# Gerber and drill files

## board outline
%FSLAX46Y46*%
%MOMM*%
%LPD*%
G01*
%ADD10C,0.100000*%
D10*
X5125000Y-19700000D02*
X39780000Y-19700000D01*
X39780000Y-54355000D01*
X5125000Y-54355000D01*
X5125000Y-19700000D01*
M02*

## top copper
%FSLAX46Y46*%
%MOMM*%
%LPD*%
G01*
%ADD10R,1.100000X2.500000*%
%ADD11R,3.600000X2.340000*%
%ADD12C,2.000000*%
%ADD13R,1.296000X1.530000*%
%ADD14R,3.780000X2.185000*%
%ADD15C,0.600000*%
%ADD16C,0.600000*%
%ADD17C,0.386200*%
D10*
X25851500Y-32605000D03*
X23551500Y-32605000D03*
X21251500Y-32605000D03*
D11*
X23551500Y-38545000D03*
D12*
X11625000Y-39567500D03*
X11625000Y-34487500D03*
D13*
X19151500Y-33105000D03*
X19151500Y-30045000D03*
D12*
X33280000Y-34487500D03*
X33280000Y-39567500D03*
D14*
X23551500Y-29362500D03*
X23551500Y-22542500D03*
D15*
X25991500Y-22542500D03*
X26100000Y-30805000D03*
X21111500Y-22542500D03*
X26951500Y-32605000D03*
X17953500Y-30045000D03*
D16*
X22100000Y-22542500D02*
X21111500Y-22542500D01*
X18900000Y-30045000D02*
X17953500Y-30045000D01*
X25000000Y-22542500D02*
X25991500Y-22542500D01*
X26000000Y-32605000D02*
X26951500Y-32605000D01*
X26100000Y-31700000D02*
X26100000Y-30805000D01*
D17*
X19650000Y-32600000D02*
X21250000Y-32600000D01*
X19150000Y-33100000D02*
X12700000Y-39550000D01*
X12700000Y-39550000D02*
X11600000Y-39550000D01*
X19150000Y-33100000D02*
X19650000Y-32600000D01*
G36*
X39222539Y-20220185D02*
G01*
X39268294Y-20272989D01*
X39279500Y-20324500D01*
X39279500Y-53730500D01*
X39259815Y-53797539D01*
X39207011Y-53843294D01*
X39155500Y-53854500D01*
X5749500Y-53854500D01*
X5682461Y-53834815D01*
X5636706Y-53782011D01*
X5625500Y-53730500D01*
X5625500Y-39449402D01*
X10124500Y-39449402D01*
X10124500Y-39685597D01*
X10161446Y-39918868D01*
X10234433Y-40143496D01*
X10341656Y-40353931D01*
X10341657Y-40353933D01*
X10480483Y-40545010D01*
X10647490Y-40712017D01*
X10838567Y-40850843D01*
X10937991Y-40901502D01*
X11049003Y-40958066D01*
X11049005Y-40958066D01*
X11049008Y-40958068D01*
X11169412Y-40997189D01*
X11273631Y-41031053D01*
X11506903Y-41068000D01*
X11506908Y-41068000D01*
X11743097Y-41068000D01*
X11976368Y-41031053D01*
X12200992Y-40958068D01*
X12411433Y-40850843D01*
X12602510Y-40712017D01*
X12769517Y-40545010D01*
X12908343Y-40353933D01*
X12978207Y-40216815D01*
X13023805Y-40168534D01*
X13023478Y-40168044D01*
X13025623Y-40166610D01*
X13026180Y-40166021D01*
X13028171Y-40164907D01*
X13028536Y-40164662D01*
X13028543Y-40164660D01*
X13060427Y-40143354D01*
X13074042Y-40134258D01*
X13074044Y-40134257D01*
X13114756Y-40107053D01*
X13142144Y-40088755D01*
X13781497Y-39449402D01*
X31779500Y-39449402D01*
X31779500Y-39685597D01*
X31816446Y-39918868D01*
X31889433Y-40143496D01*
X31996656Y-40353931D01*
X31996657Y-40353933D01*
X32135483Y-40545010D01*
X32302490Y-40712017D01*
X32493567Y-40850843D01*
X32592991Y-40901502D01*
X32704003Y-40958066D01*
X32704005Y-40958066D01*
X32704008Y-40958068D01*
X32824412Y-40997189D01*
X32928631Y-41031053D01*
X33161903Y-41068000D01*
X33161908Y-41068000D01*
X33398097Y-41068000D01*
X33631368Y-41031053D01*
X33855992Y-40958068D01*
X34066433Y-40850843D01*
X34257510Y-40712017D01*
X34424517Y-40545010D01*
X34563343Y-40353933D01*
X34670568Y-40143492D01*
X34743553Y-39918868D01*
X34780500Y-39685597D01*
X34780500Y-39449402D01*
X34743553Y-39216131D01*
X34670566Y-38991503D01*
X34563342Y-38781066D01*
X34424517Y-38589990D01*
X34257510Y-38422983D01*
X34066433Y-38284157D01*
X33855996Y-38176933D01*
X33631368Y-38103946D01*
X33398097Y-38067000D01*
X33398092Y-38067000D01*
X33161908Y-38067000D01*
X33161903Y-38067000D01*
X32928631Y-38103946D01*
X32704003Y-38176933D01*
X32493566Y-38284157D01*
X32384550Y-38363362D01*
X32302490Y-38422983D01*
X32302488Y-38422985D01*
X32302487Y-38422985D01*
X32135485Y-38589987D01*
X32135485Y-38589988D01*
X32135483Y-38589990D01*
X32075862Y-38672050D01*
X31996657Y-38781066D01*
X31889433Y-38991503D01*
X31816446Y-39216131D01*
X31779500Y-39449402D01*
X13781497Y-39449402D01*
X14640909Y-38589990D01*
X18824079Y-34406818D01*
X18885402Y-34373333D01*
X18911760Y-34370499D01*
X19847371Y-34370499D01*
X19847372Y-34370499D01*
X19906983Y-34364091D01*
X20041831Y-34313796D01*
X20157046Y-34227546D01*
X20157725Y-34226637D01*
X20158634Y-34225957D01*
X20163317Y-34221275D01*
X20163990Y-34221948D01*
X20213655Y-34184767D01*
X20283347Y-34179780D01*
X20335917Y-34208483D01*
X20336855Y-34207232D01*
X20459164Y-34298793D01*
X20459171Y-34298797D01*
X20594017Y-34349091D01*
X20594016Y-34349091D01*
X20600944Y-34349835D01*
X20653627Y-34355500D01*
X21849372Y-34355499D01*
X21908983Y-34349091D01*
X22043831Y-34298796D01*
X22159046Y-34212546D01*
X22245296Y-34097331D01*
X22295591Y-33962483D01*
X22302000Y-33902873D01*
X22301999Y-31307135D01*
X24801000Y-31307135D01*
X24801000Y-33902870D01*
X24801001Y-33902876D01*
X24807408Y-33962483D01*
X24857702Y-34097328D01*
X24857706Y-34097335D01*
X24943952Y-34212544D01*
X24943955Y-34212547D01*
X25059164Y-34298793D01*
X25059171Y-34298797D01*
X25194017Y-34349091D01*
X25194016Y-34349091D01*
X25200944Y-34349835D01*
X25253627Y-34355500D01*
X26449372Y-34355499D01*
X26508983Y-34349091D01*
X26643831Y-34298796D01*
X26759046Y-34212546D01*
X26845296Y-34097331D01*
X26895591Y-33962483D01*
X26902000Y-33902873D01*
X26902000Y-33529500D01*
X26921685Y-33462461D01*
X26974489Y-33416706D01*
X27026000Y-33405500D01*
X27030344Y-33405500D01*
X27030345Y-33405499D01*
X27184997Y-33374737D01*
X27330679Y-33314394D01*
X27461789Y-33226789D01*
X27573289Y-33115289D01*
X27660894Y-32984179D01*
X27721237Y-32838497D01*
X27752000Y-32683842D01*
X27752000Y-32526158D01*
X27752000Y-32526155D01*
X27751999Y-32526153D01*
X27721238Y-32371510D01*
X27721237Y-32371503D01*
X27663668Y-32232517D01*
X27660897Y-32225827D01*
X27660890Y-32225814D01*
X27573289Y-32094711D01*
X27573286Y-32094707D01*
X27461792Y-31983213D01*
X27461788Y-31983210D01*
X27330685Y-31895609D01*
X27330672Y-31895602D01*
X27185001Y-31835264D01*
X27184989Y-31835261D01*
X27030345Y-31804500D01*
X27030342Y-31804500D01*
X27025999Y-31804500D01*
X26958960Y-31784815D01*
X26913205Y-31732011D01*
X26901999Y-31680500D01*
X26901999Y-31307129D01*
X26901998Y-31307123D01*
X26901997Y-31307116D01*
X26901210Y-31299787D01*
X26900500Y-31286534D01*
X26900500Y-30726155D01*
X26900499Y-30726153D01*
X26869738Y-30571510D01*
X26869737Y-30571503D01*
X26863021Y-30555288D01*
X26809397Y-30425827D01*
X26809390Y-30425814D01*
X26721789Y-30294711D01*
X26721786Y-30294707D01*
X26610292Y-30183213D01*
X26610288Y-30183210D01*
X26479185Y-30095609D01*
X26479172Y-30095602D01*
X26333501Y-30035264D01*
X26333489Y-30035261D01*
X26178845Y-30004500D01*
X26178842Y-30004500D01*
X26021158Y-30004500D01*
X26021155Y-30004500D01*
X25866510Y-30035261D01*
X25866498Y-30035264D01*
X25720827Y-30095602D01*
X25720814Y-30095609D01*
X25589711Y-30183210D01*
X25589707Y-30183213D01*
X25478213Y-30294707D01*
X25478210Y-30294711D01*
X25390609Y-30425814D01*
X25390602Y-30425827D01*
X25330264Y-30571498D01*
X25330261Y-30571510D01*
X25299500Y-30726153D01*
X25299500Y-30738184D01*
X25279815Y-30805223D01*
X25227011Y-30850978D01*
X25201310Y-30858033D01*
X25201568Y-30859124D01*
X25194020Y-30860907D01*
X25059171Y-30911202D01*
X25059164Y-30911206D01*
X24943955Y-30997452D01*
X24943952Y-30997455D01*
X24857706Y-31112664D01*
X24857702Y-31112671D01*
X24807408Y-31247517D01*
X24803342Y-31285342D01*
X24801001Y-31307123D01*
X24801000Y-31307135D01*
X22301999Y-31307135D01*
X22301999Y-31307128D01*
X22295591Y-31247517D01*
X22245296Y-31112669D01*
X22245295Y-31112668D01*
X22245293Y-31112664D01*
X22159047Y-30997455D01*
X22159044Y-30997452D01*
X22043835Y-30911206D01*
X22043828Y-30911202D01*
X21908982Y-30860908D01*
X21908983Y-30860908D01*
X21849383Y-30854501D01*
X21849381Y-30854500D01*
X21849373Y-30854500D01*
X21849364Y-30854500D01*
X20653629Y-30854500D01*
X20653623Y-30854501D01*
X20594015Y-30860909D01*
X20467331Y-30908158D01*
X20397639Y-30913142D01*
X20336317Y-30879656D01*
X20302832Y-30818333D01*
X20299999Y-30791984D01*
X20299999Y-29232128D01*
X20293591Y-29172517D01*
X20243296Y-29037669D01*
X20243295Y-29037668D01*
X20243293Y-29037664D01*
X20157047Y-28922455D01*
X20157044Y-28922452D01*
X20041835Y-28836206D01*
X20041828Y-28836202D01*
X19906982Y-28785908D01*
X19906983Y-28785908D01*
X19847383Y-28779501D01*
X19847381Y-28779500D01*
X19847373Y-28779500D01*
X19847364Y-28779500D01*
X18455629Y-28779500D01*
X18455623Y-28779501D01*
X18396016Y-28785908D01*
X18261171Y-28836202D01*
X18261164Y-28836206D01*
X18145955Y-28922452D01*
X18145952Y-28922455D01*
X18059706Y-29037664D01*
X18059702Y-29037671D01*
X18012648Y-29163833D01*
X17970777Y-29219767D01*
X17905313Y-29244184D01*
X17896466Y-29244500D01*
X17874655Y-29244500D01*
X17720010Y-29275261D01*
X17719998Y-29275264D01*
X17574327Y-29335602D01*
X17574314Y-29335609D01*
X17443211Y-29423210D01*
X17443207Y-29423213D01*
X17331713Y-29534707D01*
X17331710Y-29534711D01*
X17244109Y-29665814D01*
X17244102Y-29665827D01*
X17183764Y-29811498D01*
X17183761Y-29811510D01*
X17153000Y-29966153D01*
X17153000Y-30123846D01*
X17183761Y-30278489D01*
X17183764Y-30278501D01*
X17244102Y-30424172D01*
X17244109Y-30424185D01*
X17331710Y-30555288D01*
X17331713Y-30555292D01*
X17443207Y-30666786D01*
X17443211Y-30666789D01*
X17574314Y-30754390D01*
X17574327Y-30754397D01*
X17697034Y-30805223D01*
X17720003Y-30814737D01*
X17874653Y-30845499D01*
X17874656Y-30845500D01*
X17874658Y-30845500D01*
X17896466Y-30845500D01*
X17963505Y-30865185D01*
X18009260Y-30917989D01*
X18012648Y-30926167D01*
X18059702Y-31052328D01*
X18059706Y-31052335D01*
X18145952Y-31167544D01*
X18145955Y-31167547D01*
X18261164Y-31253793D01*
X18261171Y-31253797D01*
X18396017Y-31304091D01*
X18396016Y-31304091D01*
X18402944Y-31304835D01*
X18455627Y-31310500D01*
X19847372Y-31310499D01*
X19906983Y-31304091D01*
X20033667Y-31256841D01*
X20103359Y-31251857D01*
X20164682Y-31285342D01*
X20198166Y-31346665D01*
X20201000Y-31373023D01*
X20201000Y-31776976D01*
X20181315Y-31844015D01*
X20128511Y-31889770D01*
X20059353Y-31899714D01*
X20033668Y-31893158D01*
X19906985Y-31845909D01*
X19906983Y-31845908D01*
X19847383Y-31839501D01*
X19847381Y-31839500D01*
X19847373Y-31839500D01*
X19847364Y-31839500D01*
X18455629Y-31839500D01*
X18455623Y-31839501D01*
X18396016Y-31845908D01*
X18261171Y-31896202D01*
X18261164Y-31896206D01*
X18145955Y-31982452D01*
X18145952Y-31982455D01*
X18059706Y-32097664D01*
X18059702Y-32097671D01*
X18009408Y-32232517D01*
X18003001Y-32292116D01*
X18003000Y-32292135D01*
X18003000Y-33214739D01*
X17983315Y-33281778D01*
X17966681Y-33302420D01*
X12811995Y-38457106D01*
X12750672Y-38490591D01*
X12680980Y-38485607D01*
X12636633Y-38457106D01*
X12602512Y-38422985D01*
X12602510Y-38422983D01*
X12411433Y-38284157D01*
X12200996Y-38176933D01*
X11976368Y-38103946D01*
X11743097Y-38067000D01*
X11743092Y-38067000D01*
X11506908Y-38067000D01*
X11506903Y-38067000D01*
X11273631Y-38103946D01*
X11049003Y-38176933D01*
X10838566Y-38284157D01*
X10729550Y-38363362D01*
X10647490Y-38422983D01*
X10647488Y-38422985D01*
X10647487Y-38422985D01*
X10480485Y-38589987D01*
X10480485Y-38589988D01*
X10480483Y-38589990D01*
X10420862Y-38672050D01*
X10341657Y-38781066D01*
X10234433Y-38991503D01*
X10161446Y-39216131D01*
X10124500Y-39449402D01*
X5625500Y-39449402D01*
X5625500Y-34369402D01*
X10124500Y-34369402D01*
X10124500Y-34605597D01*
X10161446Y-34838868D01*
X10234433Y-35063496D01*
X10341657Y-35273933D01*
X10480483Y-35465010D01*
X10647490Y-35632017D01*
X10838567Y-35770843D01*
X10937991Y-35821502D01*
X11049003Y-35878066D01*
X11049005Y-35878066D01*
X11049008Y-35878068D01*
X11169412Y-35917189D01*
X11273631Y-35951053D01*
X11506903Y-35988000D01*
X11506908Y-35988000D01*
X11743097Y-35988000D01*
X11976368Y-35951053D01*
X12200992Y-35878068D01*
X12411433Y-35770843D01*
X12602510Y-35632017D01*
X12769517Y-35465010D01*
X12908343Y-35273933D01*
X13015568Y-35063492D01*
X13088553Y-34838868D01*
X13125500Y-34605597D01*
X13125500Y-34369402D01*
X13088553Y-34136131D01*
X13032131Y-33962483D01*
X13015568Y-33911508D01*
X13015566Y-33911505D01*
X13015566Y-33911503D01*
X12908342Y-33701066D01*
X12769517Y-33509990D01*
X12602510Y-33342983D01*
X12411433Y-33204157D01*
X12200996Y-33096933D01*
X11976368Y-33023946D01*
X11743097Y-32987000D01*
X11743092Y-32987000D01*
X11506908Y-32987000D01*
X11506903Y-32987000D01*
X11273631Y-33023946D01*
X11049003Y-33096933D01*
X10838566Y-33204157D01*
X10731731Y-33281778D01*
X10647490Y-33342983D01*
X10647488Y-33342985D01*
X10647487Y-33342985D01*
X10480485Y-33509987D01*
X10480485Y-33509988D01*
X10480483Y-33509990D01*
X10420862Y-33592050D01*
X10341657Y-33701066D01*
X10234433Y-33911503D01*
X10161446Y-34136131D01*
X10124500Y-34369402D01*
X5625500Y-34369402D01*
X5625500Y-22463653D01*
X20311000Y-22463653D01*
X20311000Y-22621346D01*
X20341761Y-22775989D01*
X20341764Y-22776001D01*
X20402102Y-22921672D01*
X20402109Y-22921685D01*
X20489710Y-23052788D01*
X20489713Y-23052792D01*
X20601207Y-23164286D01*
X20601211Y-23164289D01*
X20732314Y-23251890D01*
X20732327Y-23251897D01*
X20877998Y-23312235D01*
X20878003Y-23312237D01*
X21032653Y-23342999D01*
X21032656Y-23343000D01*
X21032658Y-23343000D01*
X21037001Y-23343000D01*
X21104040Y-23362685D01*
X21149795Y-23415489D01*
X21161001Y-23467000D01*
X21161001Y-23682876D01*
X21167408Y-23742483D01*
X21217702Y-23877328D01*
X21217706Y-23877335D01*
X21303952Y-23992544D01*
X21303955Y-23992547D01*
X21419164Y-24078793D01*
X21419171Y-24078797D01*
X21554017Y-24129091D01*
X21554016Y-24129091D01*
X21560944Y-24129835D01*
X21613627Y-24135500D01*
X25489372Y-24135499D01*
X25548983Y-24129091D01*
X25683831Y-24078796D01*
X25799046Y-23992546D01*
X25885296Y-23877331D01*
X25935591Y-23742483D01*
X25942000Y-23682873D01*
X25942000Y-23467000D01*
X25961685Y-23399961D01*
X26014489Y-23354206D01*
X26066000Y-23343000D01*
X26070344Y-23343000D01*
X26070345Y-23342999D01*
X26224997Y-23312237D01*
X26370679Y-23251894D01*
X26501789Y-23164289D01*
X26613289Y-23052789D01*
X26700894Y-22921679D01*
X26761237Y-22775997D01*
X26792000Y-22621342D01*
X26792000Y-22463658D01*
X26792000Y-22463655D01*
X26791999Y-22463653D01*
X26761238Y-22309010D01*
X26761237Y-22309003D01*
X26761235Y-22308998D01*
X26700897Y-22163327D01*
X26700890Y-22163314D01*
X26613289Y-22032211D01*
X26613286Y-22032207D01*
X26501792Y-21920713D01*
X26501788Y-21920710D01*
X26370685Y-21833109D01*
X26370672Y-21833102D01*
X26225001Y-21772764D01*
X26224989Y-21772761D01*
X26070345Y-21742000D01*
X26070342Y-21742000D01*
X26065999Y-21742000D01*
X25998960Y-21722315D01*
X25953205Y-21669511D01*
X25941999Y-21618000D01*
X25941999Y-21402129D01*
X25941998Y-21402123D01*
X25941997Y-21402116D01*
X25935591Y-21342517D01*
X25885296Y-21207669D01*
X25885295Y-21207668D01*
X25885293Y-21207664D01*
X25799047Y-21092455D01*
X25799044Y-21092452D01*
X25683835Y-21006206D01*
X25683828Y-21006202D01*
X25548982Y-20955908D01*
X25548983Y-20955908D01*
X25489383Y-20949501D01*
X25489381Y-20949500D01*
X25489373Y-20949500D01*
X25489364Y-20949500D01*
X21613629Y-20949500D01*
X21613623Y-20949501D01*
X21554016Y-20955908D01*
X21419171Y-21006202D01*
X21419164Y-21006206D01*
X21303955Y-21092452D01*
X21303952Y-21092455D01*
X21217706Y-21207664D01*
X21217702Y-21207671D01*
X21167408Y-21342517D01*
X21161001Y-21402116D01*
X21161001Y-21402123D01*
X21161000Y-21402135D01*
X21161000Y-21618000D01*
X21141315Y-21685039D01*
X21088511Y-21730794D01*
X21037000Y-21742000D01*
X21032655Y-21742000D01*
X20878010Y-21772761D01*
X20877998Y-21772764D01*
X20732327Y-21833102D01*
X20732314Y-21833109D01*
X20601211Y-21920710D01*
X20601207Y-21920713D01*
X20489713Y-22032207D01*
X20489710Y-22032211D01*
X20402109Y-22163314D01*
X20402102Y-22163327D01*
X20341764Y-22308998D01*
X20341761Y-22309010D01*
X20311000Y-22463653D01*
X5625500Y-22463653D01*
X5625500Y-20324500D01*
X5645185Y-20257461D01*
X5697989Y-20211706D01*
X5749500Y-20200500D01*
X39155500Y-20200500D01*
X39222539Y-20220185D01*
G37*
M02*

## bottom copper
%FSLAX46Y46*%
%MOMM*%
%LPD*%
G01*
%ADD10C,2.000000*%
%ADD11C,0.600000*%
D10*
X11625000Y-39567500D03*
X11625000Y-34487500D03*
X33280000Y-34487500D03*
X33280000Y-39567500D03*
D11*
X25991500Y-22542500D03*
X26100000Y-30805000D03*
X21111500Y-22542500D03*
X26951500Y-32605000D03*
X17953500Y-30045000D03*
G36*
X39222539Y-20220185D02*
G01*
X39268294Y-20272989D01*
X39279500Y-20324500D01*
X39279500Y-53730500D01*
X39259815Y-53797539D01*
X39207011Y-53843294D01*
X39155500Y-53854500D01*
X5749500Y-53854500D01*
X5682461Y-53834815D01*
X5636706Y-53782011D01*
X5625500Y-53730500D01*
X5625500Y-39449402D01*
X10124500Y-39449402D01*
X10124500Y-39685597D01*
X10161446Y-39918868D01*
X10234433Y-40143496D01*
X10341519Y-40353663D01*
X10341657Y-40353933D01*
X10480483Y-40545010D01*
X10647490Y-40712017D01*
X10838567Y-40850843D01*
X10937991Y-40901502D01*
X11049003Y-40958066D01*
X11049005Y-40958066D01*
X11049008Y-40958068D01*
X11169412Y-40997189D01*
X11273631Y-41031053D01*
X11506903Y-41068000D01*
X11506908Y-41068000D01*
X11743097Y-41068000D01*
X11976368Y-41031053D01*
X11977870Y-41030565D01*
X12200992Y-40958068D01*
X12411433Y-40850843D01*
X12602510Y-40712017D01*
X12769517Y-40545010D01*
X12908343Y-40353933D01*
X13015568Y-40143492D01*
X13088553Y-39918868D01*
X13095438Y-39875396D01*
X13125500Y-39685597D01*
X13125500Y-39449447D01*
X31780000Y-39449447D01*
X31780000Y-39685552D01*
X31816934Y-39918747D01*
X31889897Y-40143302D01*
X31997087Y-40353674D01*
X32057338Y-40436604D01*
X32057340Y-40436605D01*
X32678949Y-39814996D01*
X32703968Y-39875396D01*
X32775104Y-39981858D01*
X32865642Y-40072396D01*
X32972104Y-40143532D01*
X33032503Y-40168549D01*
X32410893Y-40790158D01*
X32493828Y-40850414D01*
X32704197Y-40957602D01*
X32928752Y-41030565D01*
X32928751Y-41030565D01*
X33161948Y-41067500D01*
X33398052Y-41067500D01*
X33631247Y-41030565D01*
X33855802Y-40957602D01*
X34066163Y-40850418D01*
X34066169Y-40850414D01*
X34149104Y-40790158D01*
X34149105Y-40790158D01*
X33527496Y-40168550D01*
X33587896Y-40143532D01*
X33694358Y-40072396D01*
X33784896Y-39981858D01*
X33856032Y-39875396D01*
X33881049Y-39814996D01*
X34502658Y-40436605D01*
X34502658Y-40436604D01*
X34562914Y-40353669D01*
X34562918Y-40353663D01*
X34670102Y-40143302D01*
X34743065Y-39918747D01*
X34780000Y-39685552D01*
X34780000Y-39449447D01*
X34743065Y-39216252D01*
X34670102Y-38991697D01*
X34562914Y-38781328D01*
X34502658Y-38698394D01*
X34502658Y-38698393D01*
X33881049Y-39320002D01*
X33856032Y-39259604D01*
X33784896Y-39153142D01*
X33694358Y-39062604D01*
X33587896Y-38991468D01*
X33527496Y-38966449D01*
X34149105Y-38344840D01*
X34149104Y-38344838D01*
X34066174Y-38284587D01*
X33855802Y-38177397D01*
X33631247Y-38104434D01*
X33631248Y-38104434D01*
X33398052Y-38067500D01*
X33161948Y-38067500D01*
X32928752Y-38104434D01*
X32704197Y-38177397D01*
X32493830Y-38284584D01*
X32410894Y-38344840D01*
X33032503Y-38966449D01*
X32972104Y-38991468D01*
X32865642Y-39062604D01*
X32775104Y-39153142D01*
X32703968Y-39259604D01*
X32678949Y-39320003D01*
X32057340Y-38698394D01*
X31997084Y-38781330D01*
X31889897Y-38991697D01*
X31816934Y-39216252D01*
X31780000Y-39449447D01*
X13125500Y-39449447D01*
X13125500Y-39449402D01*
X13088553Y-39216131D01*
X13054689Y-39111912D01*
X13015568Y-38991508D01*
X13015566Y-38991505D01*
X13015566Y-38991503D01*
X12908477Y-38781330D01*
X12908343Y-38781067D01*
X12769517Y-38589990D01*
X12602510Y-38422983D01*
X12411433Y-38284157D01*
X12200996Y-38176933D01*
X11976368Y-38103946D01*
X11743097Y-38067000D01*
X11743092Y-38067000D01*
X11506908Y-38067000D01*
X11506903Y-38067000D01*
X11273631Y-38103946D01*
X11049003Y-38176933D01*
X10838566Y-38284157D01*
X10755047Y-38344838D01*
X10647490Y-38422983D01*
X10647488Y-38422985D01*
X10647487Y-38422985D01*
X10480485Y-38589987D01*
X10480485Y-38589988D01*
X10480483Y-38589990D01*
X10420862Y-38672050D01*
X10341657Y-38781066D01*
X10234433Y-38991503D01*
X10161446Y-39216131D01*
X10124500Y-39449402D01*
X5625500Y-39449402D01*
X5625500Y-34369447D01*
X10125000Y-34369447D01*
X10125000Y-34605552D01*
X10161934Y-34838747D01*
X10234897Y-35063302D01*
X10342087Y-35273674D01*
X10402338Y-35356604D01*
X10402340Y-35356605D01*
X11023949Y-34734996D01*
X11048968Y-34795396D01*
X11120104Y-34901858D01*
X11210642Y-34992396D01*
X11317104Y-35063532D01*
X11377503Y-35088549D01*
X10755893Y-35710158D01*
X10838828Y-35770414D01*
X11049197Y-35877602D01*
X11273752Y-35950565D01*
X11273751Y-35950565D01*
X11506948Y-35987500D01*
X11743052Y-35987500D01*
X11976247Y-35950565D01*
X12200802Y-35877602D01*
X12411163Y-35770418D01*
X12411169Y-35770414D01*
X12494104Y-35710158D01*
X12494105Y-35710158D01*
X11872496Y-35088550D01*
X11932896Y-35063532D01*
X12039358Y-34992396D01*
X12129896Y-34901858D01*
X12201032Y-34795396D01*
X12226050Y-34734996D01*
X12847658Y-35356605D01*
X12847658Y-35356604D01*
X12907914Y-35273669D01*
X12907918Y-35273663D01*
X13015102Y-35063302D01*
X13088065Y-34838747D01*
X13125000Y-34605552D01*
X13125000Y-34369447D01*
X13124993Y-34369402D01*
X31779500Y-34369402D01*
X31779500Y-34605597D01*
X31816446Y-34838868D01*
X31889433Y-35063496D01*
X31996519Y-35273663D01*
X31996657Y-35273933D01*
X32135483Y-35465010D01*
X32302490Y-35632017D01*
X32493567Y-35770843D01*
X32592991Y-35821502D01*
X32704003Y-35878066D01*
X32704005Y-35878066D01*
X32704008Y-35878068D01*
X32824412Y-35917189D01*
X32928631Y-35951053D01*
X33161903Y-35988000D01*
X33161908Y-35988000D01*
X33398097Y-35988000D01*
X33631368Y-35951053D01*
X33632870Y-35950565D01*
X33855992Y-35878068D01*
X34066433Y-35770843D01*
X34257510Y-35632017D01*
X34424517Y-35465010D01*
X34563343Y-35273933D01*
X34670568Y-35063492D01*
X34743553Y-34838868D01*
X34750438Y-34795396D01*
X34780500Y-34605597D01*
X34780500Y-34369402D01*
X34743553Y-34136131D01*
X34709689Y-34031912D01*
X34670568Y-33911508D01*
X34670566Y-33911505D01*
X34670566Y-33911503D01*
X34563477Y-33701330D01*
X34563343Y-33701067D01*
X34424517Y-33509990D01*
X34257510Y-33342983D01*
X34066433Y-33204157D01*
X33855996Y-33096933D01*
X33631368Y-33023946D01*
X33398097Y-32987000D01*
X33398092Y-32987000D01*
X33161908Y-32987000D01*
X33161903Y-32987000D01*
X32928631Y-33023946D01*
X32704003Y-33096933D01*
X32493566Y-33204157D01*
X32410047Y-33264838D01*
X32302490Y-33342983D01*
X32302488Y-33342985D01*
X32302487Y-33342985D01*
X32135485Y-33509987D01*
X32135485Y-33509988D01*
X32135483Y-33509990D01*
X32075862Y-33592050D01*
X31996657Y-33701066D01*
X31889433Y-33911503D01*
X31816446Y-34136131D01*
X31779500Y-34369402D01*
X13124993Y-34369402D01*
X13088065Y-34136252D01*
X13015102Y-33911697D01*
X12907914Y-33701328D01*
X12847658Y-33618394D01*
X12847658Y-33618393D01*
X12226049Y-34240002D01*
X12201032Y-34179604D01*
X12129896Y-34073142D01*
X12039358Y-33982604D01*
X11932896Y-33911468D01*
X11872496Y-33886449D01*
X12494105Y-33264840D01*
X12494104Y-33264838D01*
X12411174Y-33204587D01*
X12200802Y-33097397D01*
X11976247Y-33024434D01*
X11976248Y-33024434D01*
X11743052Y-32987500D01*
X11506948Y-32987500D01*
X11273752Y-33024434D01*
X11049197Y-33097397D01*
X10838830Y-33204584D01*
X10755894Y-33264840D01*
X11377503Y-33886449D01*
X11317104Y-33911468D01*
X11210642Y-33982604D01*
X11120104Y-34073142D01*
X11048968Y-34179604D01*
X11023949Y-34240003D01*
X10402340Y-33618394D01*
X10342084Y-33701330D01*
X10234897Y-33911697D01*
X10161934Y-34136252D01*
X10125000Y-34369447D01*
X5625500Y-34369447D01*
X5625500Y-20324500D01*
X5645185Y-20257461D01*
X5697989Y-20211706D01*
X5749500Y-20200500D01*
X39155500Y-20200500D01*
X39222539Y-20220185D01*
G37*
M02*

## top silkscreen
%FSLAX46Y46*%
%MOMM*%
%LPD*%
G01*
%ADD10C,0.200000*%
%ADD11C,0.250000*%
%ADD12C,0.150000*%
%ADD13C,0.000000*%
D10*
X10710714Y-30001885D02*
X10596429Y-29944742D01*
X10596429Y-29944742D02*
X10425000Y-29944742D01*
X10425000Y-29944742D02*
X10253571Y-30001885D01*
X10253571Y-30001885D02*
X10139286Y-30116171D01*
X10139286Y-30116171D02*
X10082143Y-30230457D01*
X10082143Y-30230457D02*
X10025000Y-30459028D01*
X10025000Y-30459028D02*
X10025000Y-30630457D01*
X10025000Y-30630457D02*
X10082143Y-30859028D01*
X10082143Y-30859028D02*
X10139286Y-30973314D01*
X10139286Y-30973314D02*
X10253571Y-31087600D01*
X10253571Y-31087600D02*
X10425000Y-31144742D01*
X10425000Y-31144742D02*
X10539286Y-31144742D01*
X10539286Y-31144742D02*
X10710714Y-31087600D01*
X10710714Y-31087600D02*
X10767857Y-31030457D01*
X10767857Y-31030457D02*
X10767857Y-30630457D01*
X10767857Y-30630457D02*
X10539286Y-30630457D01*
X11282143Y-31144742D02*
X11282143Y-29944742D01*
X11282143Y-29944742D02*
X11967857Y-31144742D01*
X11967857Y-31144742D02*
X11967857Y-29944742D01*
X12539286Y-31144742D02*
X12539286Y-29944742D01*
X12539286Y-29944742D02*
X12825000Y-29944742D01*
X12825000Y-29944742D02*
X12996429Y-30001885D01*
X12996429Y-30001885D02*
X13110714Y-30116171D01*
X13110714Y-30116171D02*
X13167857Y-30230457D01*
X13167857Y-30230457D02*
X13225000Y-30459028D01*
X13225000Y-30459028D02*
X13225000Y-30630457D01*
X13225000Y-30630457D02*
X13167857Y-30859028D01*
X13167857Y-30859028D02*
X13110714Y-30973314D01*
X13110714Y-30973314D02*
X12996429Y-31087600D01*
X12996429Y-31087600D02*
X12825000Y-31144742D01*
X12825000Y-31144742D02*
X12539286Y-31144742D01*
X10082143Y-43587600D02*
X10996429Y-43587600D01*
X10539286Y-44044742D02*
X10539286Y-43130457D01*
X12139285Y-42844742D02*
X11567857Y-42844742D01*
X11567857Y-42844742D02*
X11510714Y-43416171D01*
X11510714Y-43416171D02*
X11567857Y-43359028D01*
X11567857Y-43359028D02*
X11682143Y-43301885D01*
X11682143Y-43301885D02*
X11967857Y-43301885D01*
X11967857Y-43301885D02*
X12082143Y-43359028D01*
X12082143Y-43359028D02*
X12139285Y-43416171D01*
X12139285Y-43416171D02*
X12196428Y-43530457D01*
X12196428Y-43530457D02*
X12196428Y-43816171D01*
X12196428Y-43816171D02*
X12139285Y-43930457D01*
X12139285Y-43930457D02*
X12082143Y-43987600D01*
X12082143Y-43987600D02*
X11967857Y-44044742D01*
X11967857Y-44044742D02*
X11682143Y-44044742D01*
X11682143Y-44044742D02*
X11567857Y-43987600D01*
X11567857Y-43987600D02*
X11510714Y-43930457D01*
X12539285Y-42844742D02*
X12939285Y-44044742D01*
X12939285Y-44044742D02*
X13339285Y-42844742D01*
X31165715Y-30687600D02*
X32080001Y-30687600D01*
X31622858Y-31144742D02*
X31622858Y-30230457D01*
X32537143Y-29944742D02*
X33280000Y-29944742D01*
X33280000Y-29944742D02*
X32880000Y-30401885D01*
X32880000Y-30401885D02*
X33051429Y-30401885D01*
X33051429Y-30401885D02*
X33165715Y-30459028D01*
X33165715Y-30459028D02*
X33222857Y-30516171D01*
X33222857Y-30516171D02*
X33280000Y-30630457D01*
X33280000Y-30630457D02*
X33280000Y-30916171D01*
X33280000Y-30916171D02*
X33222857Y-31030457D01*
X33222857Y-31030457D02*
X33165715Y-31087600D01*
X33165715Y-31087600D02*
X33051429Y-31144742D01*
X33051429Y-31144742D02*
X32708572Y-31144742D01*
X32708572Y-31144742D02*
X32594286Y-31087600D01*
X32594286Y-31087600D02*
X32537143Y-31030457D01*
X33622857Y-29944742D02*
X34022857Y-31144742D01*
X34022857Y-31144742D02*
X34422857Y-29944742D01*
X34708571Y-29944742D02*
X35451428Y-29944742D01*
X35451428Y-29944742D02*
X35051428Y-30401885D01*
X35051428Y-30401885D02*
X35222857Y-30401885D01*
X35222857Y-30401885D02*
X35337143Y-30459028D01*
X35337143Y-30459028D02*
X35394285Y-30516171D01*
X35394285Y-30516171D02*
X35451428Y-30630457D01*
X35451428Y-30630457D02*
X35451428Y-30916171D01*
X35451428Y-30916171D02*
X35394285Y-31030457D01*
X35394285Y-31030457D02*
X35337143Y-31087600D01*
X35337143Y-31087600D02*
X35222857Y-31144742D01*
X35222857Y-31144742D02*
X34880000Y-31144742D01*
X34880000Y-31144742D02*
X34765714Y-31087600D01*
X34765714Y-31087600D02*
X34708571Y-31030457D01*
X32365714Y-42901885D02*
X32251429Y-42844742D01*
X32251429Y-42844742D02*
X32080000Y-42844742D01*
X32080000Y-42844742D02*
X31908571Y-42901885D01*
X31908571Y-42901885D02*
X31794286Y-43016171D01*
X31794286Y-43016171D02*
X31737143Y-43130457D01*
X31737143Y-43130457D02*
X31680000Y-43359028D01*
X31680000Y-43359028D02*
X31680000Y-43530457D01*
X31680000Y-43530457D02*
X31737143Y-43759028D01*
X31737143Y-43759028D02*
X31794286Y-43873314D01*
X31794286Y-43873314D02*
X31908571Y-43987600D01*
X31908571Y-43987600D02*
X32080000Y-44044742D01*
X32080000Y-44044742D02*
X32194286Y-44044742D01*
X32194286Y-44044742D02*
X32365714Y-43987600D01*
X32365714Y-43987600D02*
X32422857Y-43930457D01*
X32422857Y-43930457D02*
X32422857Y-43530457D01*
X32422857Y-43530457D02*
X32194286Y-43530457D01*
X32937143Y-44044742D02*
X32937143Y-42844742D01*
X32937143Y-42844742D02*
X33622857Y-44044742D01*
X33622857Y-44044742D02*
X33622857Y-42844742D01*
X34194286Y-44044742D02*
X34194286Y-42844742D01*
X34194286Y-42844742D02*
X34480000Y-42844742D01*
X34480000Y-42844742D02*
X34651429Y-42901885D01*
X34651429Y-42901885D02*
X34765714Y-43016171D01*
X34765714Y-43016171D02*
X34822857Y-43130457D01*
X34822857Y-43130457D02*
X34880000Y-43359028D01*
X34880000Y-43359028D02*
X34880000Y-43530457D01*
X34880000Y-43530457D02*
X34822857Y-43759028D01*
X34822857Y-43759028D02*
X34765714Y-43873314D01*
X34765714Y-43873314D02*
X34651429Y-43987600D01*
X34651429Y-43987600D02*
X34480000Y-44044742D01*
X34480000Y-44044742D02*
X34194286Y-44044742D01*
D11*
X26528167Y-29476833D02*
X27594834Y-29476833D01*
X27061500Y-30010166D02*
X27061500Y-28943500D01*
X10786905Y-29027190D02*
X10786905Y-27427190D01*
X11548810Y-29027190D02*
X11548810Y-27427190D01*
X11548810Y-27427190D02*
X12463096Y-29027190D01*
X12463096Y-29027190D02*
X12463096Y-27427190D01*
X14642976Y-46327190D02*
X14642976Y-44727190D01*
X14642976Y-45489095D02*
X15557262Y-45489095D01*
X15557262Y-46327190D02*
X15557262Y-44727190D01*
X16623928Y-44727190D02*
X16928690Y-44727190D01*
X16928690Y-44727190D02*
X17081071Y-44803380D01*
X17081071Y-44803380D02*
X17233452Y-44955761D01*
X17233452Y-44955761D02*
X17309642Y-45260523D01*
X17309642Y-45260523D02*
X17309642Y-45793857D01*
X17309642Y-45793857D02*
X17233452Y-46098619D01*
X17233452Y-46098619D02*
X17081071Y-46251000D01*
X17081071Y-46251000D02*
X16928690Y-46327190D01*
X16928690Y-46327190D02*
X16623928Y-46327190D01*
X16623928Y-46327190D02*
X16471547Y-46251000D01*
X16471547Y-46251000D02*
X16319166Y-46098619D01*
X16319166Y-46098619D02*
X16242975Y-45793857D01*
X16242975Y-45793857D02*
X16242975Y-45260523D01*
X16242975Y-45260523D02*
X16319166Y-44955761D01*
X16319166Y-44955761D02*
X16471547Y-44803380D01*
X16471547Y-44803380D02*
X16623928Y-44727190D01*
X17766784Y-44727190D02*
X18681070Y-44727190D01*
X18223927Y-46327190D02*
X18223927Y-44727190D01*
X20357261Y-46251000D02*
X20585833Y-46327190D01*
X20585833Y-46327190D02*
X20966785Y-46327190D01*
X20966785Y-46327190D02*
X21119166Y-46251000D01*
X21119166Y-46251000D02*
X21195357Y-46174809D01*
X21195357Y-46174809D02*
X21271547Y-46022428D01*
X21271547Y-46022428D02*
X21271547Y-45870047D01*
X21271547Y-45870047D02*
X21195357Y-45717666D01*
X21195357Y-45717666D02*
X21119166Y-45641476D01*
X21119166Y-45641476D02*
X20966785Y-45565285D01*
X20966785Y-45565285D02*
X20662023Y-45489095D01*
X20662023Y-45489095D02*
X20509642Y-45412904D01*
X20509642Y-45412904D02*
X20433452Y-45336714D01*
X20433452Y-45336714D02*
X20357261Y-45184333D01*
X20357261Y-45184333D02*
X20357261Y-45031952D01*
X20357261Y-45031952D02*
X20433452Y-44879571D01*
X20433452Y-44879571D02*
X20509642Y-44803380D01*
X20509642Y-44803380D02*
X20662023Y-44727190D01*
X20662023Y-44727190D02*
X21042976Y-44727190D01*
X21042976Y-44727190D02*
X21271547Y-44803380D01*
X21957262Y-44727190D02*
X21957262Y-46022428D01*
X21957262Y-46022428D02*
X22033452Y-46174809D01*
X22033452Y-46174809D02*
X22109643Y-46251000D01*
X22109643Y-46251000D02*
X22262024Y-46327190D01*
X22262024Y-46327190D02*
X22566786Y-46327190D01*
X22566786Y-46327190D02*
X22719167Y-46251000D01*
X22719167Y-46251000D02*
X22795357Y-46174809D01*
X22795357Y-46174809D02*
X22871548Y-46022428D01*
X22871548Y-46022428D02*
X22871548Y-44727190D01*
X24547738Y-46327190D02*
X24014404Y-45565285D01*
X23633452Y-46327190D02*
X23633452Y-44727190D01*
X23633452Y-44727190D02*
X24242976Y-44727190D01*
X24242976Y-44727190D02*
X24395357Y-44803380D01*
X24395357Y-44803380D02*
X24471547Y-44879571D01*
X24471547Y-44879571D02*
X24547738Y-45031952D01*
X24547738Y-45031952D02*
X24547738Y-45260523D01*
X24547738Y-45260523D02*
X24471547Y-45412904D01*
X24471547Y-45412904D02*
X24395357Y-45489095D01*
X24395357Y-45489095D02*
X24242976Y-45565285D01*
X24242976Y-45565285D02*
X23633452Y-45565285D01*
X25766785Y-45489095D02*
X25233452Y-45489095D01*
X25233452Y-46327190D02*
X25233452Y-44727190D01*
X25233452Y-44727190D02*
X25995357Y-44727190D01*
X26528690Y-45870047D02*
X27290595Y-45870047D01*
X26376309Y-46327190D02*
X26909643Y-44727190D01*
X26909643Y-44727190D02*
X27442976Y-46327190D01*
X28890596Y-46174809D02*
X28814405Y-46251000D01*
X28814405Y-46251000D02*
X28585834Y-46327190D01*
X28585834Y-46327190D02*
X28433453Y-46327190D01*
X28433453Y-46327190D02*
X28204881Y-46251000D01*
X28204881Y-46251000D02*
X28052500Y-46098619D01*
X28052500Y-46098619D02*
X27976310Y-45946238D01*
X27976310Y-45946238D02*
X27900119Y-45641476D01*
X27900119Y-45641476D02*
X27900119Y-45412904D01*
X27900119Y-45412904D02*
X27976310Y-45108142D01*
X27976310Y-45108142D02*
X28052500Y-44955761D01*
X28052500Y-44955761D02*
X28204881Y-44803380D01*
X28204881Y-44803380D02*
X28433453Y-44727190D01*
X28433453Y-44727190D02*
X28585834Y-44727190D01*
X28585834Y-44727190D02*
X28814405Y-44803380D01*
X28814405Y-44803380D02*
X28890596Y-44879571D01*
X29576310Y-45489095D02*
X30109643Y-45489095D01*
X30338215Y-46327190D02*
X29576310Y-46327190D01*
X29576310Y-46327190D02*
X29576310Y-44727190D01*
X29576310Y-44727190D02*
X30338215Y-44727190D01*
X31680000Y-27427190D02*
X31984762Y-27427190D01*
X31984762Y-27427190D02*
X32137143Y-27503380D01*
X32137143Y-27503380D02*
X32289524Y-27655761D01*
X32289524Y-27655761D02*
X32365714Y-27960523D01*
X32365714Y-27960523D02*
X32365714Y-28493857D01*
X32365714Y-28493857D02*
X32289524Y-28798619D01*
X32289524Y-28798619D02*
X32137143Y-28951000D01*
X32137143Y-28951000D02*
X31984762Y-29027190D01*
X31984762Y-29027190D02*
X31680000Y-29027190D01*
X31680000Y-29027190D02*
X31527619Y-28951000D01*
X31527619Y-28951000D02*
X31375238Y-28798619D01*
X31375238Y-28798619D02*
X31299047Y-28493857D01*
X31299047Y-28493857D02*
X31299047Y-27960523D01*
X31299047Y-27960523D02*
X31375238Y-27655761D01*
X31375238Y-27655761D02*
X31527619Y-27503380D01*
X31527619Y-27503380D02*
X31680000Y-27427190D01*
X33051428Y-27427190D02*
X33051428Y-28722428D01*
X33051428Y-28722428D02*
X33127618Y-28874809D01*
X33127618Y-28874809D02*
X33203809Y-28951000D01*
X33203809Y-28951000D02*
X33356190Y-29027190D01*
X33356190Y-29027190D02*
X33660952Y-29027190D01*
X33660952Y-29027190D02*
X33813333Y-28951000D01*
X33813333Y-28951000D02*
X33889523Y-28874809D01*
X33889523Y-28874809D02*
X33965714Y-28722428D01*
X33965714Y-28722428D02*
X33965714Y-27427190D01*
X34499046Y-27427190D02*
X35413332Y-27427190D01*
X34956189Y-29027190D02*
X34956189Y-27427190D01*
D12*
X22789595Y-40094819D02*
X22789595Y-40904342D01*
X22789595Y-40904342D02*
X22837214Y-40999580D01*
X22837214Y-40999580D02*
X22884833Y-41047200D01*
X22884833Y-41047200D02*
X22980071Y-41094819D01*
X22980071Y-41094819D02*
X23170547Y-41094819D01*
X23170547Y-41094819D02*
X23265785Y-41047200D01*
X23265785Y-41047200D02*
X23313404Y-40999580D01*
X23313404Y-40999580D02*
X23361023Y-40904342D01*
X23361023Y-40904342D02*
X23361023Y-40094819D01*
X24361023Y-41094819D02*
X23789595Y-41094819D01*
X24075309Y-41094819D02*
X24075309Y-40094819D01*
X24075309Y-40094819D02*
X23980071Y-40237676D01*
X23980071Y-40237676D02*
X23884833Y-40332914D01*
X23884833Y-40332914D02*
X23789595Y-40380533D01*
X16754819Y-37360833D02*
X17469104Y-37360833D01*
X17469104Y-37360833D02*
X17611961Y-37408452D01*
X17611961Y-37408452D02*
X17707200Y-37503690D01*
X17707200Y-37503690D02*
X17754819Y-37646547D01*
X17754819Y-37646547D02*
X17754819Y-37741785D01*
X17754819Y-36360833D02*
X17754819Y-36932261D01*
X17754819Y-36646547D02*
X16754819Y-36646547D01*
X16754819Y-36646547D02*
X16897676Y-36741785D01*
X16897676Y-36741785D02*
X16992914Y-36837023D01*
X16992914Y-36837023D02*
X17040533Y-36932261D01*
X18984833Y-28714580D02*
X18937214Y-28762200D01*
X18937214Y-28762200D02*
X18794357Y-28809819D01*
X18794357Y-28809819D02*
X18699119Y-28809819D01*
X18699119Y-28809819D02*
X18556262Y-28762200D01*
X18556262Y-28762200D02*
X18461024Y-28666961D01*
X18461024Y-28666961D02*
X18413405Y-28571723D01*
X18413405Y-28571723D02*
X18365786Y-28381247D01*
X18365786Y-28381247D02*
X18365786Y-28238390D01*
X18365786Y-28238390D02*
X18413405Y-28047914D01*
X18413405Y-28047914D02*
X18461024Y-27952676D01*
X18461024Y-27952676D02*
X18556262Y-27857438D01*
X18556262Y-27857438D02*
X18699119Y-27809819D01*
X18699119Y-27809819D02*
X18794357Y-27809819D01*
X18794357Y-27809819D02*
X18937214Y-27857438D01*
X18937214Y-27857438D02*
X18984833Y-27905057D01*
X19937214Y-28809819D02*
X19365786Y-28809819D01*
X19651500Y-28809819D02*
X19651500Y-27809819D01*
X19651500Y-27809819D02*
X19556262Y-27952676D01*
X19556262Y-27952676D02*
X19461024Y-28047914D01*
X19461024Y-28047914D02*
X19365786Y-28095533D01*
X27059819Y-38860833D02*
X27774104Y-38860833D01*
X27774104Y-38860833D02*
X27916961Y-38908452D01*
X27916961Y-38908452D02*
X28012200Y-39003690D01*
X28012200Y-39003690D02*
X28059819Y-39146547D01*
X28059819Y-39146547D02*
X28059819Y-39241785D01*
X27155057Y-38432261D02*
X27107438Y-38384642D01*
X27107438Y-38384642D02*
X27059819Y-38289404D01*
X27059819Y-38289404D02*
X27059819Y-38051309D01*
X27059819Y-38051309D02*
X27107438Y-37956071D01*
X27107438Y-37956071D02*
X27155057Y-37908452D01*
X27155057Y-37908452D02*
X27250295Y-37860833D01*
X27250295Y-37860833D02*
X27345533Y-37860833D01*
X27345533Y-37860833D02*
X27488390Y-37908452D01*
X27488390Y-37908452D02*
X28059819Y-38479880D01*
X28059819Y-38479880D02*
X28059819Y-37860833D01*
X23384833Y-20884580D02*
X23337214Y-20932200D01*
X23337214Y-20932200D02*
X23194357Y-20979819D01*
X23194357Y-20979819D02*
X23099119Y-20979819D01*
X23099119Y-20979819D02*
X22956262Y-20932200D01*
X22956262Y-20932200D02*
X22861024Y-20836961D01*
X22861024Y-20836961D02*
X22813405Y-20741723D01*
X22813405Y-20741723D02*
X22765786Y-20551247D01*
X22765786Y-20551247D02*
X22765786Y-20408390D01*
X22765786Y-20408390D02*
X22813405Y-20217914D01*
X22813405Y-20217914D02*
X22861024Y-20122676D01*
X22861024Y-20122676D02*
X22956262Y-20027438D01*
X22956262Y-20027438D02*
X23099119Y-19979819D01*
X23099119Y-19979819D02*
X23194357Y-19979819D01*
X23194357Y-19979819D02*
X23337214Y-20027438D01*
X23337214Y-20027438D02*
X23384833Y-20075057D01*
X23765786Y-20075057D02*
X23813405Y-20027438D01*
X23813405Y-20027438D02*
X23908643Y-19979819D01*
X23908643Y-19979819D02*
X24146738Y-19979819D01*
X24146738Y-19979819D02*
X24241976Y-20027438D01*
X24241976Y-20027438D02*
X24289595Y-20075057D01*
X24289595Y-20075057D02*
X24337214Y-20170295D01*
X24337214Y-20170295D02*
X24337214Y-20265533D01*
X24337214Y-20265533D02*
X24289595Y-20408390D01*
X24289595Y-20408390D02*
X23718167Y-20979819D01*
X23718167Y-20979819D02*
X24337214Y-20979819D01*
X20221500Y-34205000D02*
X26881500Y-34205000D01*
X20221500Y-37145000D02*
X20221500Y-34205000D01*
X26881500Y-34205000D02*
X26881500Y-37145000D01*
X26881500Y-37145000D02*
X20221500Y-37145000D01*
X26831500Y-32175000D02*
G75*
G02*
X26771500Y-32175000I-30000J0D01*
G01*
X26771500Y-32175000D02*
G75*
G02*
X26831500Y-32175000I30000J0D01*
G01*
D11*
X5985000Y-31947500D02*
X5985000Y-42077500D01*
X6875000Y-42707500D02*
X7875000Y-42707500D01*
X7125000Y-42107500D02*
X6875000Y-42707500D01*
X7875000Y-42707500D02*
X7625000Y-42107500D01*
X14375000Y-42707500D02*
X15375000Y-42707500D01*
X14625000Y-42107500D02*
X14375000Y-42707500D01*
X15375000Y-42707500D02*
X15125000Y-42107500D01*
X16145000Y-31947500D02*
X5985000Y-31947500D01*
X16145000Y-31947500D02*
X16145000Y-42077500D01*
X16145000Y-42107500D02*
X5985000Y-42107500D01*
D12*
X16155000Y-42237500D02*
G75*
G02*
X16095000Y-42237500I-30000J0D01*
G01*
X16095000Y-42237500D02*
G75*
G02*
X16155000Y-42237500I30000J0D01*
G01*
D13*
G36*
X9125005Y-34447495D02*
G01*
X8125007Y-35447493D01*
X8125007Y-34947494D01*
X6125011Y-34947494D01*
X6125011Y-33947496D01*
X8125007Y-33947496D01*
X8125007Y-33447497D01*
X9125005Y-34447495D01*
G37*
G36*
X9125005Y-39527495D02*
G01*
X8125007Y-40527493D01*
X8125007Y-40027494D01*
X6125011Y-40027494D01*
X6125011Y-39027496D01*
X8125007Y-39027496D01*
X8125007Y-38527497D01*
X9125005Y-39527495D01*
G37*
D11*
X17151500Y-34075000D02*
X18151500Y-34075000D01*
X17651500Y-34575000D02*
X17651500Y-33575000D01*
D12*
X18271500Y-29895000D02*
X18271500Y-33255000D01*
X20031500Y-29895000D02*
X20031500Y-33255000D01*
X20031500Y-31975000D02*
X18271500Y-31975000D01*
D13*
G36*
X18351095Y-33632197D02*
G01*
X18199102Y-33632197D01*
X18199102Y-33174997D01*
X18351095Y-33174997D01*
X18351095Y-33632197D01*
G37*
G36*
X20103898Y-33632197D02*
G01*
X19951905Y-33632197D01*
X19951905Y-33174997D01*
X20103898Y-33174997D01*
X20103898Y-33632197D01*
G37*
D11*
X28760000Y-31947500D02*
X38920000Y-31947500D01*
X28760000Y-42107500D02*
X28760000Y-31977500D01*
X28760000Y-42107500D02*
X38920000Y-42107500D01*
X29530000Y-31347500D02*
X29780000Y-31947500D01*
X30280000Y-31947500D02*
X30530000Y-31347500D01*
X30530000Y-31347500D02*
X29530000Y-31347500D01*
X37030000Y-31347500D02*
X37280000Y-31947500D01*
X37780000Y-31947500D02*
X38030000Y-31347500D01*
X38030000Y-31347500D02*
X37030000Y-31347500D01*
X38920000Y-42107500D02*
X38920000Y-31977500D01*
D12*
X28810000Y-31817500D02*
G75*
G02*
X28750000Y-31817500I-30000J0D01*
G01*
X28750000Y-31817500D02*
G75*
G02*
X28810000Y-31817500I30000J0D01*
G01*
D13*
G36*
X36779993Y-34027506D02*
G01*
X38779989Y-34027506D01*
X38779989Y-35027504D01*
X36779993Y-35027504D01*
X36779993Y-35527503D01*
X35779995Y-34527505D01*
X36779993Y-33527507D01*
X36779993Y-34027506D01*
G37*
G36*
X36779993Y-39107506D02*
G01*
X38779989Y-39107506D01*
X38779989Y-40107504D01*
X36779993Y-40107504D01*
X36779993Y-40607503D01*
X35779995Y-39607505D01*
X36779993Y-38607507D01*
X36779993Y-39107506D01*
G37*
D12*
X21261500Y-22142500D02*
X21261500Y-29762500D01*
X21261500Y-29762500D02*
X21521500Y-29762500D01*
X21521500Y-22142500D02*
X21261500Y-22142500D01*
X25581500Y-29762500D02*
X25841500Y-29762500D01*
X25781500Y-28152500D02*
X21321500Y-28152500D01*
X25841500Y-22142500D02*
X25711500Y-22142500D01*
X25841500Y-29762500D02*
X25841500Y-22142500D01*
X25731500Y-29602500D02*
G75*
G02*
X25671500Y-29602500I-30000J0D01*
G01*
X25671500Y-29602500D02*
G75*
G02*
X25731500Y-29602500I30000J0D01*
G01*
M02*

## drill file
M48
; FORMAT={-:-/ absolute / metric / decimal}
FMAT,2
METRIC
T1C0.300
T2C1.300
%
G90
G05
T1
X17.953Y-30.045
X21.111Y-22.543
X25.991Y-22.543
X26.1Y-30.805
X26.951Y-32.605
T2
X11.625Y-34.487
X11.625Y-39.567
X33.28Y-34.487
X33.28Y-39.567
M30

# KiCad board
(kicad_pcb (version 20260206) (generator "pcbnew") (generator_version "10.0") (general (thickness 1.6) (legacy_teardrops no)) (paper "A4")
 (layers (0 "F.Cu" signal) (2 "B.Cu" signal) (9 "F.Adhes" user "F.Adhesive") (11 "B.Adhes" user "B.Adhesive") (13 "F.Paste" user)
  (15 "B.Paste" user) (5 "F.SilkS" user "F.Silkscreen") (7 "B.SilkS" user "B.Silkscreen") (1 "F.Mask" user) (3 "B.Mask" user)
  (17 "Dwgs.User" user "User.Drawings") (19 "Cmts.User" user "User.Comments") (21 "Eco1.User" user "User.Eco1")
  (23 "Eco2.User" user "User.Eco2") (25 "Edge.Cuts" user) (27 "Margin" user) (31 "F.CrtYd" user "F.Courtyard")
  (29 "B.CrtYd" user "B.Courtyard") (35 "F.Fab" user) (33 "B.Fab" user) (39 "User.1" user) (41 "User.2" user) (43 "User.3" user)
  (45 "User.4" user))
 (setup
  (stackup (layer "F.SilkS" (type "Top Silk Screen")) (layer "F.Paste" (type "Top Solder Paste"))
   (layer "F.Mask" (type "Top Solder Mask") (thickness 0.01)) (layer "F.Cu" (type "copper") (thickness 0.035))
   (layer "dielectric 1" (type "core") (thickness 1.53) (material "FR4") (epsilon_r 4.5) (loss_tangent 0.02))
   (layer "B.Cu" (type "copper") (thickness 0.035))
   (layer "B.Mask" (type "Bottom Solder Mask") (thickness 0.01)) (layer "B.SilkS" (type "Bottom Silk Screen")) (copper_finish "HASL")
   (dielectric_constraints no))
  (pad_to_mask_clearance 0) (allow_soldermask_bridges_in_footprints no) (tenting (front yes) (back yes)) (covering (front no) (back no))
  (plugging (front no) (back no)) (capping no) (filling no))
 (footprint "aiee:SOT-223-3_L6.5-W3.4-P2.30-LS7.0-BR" (layer "F.Cu") (at 23.5515 35.575 90)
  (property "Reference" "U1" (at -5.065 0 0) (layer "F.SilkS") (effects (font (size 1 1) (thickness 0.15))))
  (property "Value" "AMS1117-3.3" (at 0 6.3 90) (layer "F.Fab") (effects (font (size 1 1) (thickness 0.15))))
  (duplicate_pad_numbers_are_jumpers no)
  (fp_line (start 1.37 -3.33) (end 1.37 3.33) (stroke (width 0.15) (type solid)) (layer "F.SilkS"))
  (fp_line (start -1.57 -3.33) (end 1.37 -3.33) (stroke (width 0.15) (type solid)) (layer "F.SilkS"))
  (fp_line (start 1.37 3.33) (end -1.57 3.33) (stroke (width 0.15) (type solid)) (layer "F.SilkS"))
  (fp_line (start -1.57 3.33) (end -1.57 -3.33) (stroke (width 0.15) (type solid)) (layer "F.SilkS"))
  (fp_circle (center 3.4 3.25) (end 3.43 3.25) (stroke (width 0.15) (type solid)) (fill no) (layer "F.SilkS"))
  (pad "1" smd rect (at 2.97 2.3 90) (size 2.5 1.1) (layers "F.Cu" "F.Mask" "F.Paste") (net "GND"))
  (pad "2" smd rect (at 2.97 0 90) (size 2.5 1.1) (layers "F.Cu" "F.Mask" "F.Paste") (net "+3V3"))
  (pad "3" smd rect (at 2.97 -2.3 90) (size 2.5 1.1) (layers "F.Cu" "F.Mask" "F.Paste") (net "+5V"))
  (pad "4" smd rect (at -2.97 0 90) (size 2.34 3.6) (layers "F.Cu" "F.Mask" "F.Paste") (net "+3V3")))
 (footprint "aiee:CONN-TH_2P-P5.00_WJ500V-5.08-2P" (layer "F.Cu") (at 11.625 37.0275 90)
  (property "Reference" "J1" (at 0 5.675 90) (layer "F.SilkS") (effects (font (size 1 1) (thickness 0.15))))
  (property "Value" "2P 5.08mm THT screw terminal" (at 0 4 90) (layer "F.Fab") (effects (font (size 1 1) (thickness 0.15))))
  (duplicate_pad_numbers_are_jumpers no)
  (fp_line (start 5.08 -5.64) (end -5.05 -5.64) (stroke (width 0.25) (type solid)) (layer "F.SilkS"))
  (fp_line (start -5.68 -4.75) (end -5.68 -3.75) (stroke (width 0.25) (type solid)) (layer "F.SilkS"))
  (fp_line (start -5.08 -4.5) (end -5.68 -4.75) (stroke (width 0.25) (type solid)) (layer "F.SilkS"))
  (fp_line (start -5.68 -3.75) (end -5.08 -4) (stroke (width 0.25) (type solid)) (layer "F.SilkS"))
  (fp_line (start -5.68 2.75) (end -5.68 3.75) (stroke (width 0.25) (type solid)) (layer "F.SilkS"))
  (fp_line (start -5.08 3) (end -5.68 2.75) (stroke (width 0.25) (type solid)) (layer "F.SilkS"))
  (fp_line (start -5.68 3.75) (end -5.08 3.5) (stroke (width 0.25) (type solid)) (layer "F.SilkS"))
  (fp_line (start 5.08 4.52) (end 5.08 -5.64) (stroke (width 0.25) (type solid)) (layer "F.SilkS"))
  (fp_line (start 5.08 4.52) (end -5.05 4.52) (stroke (width 0.25) (type solid)) (layer "F.SilkS"))
  (fp_line (start -5.08 4.52) (end -5.08 -5.64) (stroke (width 0.25) (type solid)) (layer "F.SilkS"))
  (fp_circle (center -5.21 4.5) (end -5.18 4.5) (stroke (width 0.15) (type solid)) (fill no) (layer "F.SilkS"))
  (fp_poly
   (pts (xy 2.080006 -5.499989) (xy 3.080004 -5.499989) (xy 3.080004 -3.499993) (xy 3.580003 -3.499993) (xy 2.580005 -2.499995)
    (xy 1.580007 -3.499993) (xy 2.080006 -3.499993) (xy 2.080006 -5.499989))
   (stroke (width 0) (type solid)) (fill yes) (layer "F.SilkS"))
  (fp_poly
   (pts (xy -2.999994 -5.499989) (xy -1.999996 -5.499989) (xy -1.999996 -3.499993) (xy -1.499997 -3.499993) (xy -2.499995 -2.499995)
    (xy -3.499993 -3.499993) (xy -2.999994 -3.499993) (xy -2.999994 -5.499989))
   (stroke (width 0) (type solid)) (fill yes) (layer "F.SilkS"))
  (pad "1" thru_hole circle (at -2.54 0 270) (size 2 2) (drill 1.300022) (layers "*.Cu" "*.Mask") (remove_unused_layers no) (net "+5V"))
  (pad "2" thru_hole circle (at 2.54 0 270) (size 2 2) (drill 1.300022) (layers "*.Cu" "*.Mask") (remove_unused_layers no) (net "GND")))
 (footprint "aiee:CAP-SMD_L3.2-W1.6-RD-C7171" (layer "F.Cu") (at 19.1515 31.575 90)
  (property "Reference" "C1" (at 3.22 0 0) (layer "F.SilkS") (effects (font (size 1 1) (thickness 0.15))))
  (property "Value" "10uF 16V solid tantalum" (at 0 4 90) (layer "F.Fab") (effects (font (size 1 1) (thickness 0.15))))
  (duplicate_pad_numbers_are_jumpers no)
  (fp_line (start -2.5 -2) (end -2.5 -1) (stroke (width 0.25) (type solid)) (layer "F.SilkS"))
  (fp_line (start -3 -1.5) (end -2 -1.5) (stroke (width 0.25) (type solid)) (layer "F.SilkS"))
  (fp_line (start 1.68 -0.88) (end -1.68 -0.88) (stroke (width 0.15) (type solid)) (layer "F.SilkS"))
  (fp_line (start 1.68 0.88) (end -1.68 0.88) (stroke (width 0.15) (type solid)) (layer "F.SilkS"))
  (fp_line (start -0.4 0.88) (end -0.4 -0.88) (stroke (width 0.15) (type solid)) (layer "F.SilkS"))
  (fp_poly
   (pts (xy -1.599997 -0.952398) (xy -1.599997 -0.800405) (xy -2.057197 -0.800405) (xy -2.057197 -0.952398) (xy -1.599997 -0.952398))
   (stroke (width 0) (type solid)) (fill yes) (layer "F.SilkS"))
  (fp_poly
   (pts (xy -1.599997 0.952398) (xy -1.599997 0.800405) (xy -2.057197 0.800405) (xy -2.057197 0.952398) (xy -1.599997 0.952398))
   (stroke (width 0) (type solid)) (fill yes) (layer "F.SilkS"))
  (pad "1" smd rect (at -1.53 0 270) (size 1.53 1.296) (layers "F.Cu" "F.Mask" "F.Paste") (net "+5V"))
  (pad "2" smd rect (at 1.53 0 270) (size 1.53 1.296) (layers "F.Cu" "F.Mask" "F.Paste") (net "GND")))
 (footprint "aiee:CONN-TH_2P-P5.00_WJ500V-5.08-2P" (layer "F.Cu") (at 33.28 37.0275 -90)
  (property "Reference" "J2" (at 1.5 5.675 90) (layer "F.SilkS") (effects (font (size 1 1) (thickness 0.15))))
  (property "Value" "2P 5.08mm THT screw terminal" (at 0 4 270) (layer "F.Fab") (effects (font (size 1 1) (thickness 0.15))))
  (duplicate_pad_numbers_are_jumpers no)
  (fp_line (start -5.08 4.52) (end -5.08 -5.64) (stroke (width 0.25) (type solid)) (layer "F.SilkS"))
  (fp_line (start 5.08 4.52) (end -5.05 4.52) (stroke (width 0.25) (type solid)) (layer "F.SilkS"))
  (fp_line (start 5.08 4.52) (end 5.08 -5.64) (stroke (width 0.25) (type solid)) (layer "F.SilkS"))
  (fp_line (start -5.68 3.75) (end -5.08 3.5) (stroke (width 0.25) (type solid)) (layer "F.SilkS"))
  (fp_line (start -5.08 3) (end -5.68 2.75) (stroke (width 0.25) (type solid)) (layer "F.SilkS"))
  (fp_line (start -5.68 2.75) (end -5.68 3.75) (stroke (width 0.25) (type solid)) (layer "F.SilkS"))
  (fp_line (start -5.68 -3.75) (end -5.08 -4) (stroke (width 0.25) (type solid)) (layer "F.SilkS"))
  (fp_line (start -5.08 -4.5) (end -5.68 -4.75) (stroke (width 0.25) (type solid)) (layer "F.SilkS"))
  (fp_line (start -5.68 -4.75) (end -5.68 -3.75) (stroke (width 0.25) (type solid)) (layer "F.SilkS"))
  (fp_line (start 5.08 -5.64) (end -5.05 -5.64) (stroke (width 0.25) (type solid)) (layer "F.SilkS"))
  (fp_circle (center -5.21 4.5) (end -5.18 4.5) (stroke (width 0.15) (type solid)) (fill no) (layer "F.SilkS"))
  (fp_poly
   (pts (xy -2.999994 -5.499989) (xy -1.999996 -5.499989) (xy -1.999996 -3.499993) (xy -1.499997 -3.499993) (xy -2.499995 -2.499995)
    (xy -3.499993 -3.499993) (xy -2.999994 -3.499993) (xy -2.999994 -5.499989))
   (stroke (width 0) (type solid)) (fill yes) (layer "F.SilkS"))
  (fp_poly
   (pts (xy 2.080006 -5.499989) (xy 3.080004 -5.499989) (xy 3.080004 -3.499993) (xy 3.580003 -3.499993) (xy 2.580005 -2.499995)
    (xy 1.580007 -3.499993) (xy 2.080006 -3.499993) (xy 2.080006 -5.499989))
   (stroke (width 0) (type solid)) (fill yes) (layer "F.SilkS"))
  (pad "1" thru_hole circle (at -2.54 0 90) (size 2 2) (drill 1.300022) (layers "*.Cu" "*.Mask") (remove_unused_layers no) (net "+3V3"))
  (pad "2" thru_hole circle (at 2.54 0 90) (size 2 2) (drill 1.300022) (layers "*.Cu" "*.Mask") (remove_unused_layers no) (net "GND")))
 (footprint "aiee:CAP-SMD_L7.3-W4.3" (layer "F.Cu") (at 23.5515 25.9525 -90)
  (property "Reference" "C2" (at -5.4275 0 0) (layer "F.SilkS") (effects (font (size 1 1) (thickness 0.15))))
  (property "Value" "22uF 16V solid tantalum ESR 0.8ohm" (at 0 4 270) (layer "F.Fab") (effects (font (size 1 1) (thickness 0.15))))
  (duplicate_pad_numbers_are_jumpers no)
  (fp_line (start -3.81 2.29) (end 3.81 2.29) (stroke (width 0.15) (type solid)) (layer "F.SilkS"))
  (fp_line (start 3.81 2.29) (end 3.81 2.03) (stroke (width 0.15) (type solid)) (layer "F.SilkS"))
  (fp_line (start -3.81 2.03) (end -3.81 2.29) (stroke (width 0.15) (type solid)) (layer "F.SilkS"))
  (fp_line (start 3.81 -2.03) (end 3.81 -2.29) (stroke (width 0.15) (type solid)) (layer "F.SilkS"))
  (fp_line (start 2.2 -2.23) (end 2.2 2.23) (stroke (width 0.15) (type solid)) (layer "F.SilkS"))
  (fp_line (start -3.81 -2.29) (end -3.81 -2.16) (stroke (width 0.15) (type solid)) (layer "F.SilkS"))
  (fp_line (start 3.81 -2.29) (end -3.81 -2.29) (stroke (width 0.15) (type solid)) (layer "F.SilkS"))
  (fp_circle (center 3.65 -2.15) (end 3.68 -2.15) (stroke (width 0.15) (type solid)) (fill no) (layer "F.SilkS"))
  (pad "1" smd rect (at 3.41 0 90) (size 2.185 3.78) (layers "F.Cu" "F.Mask" "F.Paste") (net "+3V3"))
  (pad "2" smd rect (at -3.41 0 90) (size 2.185 3.78) (layers "F.Cu" "F.Mask" "F.Paste") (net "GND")))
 (gr_rect (start 5.125 19.7) (end 39.78 54.355) (stroke (width 0.1) (type default)) (fill no) (layer "Edge.Cuts"))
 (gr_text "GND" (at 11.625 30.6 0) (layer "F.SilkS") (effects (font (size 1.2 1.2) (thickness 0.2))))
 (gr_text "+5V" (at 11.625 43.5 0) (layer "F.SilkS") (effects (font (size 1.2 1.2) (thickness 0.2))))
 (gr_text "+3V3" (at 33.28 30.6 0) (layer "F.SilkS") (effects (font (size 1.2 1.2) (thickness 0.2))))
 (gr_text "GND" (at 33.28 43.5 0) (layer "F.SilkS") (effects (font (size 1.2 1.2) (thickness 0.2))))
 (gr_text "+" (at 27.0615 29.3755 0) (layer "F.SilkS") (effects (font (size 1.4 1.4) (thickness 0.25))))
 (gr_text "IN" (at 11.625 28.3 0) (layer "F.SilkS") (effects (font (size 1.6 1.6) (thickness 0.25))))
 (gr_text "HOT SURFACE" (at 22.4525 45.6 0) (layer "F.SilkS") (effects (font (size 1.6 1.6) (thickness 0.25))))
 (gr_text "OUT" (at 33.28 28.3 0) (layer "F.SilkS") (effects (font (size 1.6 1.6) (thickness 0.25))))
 (segment (start 22.1 22.5425) (end 21.1115 22.5425) (width 0.6) (layer "F.Cu") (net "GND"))
 (segment (start 18.9 30.045) (end 17.9535 30.045) (width 0.6) (layer "F.Cu") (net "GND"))
 (segment (start 25 22.5425) (end 25.9915 22.5425) (width 0.6) (layer "F.Cu") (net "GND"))
 (segment (start 26 32.605) (end 26.9515 32.605) (width 0.6) (layer "F.Cu") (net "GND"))
 (segment (start 26.1 31.7) (end 26.1 30.805) (width 0.6) (layer "F.Cu") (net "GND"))
 (via (at 25.9915 22.5425) (size 0.6) (drill 0.3) (layers "F.Cu" "B.Cu") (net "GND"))
 (via (at 26.1 30.805) (size 0.6) (drill 0.3) (layers "F.Cu" "B.Cu") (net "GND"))
 (via (at 21.1115 22.5425) (size 0.6) (drill 0.3) (layers "F.Cu" "B.Cu") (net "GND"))
 (via (at 26.9515 32.605) (size 0.6) (drill 0.3) (layers "F.Cu" "B.Cu") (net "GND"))
 (via (at 17.9535 30.045) (size 0.6) (drill 0.3) (layers "F.Cu" "B.Cu") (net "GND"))
 (segment (start 19.65 32.6) (end 21.25 32.6) (width 0.3862) (layer "F.Cu") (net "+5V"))
 (segment (start 19.15 33.1) (end 12.7 39.55) (width 0.3862) (layer "F.Cu") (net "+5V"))
 (segment (start 12.7 39.55) (end 11.6 39.55) (width 0.3862) (layer "F.Cu") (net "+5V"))
 (segment (start 19.15 33.1) (end 19.65 32.6) (width 0.3862) (layer "F.Cu") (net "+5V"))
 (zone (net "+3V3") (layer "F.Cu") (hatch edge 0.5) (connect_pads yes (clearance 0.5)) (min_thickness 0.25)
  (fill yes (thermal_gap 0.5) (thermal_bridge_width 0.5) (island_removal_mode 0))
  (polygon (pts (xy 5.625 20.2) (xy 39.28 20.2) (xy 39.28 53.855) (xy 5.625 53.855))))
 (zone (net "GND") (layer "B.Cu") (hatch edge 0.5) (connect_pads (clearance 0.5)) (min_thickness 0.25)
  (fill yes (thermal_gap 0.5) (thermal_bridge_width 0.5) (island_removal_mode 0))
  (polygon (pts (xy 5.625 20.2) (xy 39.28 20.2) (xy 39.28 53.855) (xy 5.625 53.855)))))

